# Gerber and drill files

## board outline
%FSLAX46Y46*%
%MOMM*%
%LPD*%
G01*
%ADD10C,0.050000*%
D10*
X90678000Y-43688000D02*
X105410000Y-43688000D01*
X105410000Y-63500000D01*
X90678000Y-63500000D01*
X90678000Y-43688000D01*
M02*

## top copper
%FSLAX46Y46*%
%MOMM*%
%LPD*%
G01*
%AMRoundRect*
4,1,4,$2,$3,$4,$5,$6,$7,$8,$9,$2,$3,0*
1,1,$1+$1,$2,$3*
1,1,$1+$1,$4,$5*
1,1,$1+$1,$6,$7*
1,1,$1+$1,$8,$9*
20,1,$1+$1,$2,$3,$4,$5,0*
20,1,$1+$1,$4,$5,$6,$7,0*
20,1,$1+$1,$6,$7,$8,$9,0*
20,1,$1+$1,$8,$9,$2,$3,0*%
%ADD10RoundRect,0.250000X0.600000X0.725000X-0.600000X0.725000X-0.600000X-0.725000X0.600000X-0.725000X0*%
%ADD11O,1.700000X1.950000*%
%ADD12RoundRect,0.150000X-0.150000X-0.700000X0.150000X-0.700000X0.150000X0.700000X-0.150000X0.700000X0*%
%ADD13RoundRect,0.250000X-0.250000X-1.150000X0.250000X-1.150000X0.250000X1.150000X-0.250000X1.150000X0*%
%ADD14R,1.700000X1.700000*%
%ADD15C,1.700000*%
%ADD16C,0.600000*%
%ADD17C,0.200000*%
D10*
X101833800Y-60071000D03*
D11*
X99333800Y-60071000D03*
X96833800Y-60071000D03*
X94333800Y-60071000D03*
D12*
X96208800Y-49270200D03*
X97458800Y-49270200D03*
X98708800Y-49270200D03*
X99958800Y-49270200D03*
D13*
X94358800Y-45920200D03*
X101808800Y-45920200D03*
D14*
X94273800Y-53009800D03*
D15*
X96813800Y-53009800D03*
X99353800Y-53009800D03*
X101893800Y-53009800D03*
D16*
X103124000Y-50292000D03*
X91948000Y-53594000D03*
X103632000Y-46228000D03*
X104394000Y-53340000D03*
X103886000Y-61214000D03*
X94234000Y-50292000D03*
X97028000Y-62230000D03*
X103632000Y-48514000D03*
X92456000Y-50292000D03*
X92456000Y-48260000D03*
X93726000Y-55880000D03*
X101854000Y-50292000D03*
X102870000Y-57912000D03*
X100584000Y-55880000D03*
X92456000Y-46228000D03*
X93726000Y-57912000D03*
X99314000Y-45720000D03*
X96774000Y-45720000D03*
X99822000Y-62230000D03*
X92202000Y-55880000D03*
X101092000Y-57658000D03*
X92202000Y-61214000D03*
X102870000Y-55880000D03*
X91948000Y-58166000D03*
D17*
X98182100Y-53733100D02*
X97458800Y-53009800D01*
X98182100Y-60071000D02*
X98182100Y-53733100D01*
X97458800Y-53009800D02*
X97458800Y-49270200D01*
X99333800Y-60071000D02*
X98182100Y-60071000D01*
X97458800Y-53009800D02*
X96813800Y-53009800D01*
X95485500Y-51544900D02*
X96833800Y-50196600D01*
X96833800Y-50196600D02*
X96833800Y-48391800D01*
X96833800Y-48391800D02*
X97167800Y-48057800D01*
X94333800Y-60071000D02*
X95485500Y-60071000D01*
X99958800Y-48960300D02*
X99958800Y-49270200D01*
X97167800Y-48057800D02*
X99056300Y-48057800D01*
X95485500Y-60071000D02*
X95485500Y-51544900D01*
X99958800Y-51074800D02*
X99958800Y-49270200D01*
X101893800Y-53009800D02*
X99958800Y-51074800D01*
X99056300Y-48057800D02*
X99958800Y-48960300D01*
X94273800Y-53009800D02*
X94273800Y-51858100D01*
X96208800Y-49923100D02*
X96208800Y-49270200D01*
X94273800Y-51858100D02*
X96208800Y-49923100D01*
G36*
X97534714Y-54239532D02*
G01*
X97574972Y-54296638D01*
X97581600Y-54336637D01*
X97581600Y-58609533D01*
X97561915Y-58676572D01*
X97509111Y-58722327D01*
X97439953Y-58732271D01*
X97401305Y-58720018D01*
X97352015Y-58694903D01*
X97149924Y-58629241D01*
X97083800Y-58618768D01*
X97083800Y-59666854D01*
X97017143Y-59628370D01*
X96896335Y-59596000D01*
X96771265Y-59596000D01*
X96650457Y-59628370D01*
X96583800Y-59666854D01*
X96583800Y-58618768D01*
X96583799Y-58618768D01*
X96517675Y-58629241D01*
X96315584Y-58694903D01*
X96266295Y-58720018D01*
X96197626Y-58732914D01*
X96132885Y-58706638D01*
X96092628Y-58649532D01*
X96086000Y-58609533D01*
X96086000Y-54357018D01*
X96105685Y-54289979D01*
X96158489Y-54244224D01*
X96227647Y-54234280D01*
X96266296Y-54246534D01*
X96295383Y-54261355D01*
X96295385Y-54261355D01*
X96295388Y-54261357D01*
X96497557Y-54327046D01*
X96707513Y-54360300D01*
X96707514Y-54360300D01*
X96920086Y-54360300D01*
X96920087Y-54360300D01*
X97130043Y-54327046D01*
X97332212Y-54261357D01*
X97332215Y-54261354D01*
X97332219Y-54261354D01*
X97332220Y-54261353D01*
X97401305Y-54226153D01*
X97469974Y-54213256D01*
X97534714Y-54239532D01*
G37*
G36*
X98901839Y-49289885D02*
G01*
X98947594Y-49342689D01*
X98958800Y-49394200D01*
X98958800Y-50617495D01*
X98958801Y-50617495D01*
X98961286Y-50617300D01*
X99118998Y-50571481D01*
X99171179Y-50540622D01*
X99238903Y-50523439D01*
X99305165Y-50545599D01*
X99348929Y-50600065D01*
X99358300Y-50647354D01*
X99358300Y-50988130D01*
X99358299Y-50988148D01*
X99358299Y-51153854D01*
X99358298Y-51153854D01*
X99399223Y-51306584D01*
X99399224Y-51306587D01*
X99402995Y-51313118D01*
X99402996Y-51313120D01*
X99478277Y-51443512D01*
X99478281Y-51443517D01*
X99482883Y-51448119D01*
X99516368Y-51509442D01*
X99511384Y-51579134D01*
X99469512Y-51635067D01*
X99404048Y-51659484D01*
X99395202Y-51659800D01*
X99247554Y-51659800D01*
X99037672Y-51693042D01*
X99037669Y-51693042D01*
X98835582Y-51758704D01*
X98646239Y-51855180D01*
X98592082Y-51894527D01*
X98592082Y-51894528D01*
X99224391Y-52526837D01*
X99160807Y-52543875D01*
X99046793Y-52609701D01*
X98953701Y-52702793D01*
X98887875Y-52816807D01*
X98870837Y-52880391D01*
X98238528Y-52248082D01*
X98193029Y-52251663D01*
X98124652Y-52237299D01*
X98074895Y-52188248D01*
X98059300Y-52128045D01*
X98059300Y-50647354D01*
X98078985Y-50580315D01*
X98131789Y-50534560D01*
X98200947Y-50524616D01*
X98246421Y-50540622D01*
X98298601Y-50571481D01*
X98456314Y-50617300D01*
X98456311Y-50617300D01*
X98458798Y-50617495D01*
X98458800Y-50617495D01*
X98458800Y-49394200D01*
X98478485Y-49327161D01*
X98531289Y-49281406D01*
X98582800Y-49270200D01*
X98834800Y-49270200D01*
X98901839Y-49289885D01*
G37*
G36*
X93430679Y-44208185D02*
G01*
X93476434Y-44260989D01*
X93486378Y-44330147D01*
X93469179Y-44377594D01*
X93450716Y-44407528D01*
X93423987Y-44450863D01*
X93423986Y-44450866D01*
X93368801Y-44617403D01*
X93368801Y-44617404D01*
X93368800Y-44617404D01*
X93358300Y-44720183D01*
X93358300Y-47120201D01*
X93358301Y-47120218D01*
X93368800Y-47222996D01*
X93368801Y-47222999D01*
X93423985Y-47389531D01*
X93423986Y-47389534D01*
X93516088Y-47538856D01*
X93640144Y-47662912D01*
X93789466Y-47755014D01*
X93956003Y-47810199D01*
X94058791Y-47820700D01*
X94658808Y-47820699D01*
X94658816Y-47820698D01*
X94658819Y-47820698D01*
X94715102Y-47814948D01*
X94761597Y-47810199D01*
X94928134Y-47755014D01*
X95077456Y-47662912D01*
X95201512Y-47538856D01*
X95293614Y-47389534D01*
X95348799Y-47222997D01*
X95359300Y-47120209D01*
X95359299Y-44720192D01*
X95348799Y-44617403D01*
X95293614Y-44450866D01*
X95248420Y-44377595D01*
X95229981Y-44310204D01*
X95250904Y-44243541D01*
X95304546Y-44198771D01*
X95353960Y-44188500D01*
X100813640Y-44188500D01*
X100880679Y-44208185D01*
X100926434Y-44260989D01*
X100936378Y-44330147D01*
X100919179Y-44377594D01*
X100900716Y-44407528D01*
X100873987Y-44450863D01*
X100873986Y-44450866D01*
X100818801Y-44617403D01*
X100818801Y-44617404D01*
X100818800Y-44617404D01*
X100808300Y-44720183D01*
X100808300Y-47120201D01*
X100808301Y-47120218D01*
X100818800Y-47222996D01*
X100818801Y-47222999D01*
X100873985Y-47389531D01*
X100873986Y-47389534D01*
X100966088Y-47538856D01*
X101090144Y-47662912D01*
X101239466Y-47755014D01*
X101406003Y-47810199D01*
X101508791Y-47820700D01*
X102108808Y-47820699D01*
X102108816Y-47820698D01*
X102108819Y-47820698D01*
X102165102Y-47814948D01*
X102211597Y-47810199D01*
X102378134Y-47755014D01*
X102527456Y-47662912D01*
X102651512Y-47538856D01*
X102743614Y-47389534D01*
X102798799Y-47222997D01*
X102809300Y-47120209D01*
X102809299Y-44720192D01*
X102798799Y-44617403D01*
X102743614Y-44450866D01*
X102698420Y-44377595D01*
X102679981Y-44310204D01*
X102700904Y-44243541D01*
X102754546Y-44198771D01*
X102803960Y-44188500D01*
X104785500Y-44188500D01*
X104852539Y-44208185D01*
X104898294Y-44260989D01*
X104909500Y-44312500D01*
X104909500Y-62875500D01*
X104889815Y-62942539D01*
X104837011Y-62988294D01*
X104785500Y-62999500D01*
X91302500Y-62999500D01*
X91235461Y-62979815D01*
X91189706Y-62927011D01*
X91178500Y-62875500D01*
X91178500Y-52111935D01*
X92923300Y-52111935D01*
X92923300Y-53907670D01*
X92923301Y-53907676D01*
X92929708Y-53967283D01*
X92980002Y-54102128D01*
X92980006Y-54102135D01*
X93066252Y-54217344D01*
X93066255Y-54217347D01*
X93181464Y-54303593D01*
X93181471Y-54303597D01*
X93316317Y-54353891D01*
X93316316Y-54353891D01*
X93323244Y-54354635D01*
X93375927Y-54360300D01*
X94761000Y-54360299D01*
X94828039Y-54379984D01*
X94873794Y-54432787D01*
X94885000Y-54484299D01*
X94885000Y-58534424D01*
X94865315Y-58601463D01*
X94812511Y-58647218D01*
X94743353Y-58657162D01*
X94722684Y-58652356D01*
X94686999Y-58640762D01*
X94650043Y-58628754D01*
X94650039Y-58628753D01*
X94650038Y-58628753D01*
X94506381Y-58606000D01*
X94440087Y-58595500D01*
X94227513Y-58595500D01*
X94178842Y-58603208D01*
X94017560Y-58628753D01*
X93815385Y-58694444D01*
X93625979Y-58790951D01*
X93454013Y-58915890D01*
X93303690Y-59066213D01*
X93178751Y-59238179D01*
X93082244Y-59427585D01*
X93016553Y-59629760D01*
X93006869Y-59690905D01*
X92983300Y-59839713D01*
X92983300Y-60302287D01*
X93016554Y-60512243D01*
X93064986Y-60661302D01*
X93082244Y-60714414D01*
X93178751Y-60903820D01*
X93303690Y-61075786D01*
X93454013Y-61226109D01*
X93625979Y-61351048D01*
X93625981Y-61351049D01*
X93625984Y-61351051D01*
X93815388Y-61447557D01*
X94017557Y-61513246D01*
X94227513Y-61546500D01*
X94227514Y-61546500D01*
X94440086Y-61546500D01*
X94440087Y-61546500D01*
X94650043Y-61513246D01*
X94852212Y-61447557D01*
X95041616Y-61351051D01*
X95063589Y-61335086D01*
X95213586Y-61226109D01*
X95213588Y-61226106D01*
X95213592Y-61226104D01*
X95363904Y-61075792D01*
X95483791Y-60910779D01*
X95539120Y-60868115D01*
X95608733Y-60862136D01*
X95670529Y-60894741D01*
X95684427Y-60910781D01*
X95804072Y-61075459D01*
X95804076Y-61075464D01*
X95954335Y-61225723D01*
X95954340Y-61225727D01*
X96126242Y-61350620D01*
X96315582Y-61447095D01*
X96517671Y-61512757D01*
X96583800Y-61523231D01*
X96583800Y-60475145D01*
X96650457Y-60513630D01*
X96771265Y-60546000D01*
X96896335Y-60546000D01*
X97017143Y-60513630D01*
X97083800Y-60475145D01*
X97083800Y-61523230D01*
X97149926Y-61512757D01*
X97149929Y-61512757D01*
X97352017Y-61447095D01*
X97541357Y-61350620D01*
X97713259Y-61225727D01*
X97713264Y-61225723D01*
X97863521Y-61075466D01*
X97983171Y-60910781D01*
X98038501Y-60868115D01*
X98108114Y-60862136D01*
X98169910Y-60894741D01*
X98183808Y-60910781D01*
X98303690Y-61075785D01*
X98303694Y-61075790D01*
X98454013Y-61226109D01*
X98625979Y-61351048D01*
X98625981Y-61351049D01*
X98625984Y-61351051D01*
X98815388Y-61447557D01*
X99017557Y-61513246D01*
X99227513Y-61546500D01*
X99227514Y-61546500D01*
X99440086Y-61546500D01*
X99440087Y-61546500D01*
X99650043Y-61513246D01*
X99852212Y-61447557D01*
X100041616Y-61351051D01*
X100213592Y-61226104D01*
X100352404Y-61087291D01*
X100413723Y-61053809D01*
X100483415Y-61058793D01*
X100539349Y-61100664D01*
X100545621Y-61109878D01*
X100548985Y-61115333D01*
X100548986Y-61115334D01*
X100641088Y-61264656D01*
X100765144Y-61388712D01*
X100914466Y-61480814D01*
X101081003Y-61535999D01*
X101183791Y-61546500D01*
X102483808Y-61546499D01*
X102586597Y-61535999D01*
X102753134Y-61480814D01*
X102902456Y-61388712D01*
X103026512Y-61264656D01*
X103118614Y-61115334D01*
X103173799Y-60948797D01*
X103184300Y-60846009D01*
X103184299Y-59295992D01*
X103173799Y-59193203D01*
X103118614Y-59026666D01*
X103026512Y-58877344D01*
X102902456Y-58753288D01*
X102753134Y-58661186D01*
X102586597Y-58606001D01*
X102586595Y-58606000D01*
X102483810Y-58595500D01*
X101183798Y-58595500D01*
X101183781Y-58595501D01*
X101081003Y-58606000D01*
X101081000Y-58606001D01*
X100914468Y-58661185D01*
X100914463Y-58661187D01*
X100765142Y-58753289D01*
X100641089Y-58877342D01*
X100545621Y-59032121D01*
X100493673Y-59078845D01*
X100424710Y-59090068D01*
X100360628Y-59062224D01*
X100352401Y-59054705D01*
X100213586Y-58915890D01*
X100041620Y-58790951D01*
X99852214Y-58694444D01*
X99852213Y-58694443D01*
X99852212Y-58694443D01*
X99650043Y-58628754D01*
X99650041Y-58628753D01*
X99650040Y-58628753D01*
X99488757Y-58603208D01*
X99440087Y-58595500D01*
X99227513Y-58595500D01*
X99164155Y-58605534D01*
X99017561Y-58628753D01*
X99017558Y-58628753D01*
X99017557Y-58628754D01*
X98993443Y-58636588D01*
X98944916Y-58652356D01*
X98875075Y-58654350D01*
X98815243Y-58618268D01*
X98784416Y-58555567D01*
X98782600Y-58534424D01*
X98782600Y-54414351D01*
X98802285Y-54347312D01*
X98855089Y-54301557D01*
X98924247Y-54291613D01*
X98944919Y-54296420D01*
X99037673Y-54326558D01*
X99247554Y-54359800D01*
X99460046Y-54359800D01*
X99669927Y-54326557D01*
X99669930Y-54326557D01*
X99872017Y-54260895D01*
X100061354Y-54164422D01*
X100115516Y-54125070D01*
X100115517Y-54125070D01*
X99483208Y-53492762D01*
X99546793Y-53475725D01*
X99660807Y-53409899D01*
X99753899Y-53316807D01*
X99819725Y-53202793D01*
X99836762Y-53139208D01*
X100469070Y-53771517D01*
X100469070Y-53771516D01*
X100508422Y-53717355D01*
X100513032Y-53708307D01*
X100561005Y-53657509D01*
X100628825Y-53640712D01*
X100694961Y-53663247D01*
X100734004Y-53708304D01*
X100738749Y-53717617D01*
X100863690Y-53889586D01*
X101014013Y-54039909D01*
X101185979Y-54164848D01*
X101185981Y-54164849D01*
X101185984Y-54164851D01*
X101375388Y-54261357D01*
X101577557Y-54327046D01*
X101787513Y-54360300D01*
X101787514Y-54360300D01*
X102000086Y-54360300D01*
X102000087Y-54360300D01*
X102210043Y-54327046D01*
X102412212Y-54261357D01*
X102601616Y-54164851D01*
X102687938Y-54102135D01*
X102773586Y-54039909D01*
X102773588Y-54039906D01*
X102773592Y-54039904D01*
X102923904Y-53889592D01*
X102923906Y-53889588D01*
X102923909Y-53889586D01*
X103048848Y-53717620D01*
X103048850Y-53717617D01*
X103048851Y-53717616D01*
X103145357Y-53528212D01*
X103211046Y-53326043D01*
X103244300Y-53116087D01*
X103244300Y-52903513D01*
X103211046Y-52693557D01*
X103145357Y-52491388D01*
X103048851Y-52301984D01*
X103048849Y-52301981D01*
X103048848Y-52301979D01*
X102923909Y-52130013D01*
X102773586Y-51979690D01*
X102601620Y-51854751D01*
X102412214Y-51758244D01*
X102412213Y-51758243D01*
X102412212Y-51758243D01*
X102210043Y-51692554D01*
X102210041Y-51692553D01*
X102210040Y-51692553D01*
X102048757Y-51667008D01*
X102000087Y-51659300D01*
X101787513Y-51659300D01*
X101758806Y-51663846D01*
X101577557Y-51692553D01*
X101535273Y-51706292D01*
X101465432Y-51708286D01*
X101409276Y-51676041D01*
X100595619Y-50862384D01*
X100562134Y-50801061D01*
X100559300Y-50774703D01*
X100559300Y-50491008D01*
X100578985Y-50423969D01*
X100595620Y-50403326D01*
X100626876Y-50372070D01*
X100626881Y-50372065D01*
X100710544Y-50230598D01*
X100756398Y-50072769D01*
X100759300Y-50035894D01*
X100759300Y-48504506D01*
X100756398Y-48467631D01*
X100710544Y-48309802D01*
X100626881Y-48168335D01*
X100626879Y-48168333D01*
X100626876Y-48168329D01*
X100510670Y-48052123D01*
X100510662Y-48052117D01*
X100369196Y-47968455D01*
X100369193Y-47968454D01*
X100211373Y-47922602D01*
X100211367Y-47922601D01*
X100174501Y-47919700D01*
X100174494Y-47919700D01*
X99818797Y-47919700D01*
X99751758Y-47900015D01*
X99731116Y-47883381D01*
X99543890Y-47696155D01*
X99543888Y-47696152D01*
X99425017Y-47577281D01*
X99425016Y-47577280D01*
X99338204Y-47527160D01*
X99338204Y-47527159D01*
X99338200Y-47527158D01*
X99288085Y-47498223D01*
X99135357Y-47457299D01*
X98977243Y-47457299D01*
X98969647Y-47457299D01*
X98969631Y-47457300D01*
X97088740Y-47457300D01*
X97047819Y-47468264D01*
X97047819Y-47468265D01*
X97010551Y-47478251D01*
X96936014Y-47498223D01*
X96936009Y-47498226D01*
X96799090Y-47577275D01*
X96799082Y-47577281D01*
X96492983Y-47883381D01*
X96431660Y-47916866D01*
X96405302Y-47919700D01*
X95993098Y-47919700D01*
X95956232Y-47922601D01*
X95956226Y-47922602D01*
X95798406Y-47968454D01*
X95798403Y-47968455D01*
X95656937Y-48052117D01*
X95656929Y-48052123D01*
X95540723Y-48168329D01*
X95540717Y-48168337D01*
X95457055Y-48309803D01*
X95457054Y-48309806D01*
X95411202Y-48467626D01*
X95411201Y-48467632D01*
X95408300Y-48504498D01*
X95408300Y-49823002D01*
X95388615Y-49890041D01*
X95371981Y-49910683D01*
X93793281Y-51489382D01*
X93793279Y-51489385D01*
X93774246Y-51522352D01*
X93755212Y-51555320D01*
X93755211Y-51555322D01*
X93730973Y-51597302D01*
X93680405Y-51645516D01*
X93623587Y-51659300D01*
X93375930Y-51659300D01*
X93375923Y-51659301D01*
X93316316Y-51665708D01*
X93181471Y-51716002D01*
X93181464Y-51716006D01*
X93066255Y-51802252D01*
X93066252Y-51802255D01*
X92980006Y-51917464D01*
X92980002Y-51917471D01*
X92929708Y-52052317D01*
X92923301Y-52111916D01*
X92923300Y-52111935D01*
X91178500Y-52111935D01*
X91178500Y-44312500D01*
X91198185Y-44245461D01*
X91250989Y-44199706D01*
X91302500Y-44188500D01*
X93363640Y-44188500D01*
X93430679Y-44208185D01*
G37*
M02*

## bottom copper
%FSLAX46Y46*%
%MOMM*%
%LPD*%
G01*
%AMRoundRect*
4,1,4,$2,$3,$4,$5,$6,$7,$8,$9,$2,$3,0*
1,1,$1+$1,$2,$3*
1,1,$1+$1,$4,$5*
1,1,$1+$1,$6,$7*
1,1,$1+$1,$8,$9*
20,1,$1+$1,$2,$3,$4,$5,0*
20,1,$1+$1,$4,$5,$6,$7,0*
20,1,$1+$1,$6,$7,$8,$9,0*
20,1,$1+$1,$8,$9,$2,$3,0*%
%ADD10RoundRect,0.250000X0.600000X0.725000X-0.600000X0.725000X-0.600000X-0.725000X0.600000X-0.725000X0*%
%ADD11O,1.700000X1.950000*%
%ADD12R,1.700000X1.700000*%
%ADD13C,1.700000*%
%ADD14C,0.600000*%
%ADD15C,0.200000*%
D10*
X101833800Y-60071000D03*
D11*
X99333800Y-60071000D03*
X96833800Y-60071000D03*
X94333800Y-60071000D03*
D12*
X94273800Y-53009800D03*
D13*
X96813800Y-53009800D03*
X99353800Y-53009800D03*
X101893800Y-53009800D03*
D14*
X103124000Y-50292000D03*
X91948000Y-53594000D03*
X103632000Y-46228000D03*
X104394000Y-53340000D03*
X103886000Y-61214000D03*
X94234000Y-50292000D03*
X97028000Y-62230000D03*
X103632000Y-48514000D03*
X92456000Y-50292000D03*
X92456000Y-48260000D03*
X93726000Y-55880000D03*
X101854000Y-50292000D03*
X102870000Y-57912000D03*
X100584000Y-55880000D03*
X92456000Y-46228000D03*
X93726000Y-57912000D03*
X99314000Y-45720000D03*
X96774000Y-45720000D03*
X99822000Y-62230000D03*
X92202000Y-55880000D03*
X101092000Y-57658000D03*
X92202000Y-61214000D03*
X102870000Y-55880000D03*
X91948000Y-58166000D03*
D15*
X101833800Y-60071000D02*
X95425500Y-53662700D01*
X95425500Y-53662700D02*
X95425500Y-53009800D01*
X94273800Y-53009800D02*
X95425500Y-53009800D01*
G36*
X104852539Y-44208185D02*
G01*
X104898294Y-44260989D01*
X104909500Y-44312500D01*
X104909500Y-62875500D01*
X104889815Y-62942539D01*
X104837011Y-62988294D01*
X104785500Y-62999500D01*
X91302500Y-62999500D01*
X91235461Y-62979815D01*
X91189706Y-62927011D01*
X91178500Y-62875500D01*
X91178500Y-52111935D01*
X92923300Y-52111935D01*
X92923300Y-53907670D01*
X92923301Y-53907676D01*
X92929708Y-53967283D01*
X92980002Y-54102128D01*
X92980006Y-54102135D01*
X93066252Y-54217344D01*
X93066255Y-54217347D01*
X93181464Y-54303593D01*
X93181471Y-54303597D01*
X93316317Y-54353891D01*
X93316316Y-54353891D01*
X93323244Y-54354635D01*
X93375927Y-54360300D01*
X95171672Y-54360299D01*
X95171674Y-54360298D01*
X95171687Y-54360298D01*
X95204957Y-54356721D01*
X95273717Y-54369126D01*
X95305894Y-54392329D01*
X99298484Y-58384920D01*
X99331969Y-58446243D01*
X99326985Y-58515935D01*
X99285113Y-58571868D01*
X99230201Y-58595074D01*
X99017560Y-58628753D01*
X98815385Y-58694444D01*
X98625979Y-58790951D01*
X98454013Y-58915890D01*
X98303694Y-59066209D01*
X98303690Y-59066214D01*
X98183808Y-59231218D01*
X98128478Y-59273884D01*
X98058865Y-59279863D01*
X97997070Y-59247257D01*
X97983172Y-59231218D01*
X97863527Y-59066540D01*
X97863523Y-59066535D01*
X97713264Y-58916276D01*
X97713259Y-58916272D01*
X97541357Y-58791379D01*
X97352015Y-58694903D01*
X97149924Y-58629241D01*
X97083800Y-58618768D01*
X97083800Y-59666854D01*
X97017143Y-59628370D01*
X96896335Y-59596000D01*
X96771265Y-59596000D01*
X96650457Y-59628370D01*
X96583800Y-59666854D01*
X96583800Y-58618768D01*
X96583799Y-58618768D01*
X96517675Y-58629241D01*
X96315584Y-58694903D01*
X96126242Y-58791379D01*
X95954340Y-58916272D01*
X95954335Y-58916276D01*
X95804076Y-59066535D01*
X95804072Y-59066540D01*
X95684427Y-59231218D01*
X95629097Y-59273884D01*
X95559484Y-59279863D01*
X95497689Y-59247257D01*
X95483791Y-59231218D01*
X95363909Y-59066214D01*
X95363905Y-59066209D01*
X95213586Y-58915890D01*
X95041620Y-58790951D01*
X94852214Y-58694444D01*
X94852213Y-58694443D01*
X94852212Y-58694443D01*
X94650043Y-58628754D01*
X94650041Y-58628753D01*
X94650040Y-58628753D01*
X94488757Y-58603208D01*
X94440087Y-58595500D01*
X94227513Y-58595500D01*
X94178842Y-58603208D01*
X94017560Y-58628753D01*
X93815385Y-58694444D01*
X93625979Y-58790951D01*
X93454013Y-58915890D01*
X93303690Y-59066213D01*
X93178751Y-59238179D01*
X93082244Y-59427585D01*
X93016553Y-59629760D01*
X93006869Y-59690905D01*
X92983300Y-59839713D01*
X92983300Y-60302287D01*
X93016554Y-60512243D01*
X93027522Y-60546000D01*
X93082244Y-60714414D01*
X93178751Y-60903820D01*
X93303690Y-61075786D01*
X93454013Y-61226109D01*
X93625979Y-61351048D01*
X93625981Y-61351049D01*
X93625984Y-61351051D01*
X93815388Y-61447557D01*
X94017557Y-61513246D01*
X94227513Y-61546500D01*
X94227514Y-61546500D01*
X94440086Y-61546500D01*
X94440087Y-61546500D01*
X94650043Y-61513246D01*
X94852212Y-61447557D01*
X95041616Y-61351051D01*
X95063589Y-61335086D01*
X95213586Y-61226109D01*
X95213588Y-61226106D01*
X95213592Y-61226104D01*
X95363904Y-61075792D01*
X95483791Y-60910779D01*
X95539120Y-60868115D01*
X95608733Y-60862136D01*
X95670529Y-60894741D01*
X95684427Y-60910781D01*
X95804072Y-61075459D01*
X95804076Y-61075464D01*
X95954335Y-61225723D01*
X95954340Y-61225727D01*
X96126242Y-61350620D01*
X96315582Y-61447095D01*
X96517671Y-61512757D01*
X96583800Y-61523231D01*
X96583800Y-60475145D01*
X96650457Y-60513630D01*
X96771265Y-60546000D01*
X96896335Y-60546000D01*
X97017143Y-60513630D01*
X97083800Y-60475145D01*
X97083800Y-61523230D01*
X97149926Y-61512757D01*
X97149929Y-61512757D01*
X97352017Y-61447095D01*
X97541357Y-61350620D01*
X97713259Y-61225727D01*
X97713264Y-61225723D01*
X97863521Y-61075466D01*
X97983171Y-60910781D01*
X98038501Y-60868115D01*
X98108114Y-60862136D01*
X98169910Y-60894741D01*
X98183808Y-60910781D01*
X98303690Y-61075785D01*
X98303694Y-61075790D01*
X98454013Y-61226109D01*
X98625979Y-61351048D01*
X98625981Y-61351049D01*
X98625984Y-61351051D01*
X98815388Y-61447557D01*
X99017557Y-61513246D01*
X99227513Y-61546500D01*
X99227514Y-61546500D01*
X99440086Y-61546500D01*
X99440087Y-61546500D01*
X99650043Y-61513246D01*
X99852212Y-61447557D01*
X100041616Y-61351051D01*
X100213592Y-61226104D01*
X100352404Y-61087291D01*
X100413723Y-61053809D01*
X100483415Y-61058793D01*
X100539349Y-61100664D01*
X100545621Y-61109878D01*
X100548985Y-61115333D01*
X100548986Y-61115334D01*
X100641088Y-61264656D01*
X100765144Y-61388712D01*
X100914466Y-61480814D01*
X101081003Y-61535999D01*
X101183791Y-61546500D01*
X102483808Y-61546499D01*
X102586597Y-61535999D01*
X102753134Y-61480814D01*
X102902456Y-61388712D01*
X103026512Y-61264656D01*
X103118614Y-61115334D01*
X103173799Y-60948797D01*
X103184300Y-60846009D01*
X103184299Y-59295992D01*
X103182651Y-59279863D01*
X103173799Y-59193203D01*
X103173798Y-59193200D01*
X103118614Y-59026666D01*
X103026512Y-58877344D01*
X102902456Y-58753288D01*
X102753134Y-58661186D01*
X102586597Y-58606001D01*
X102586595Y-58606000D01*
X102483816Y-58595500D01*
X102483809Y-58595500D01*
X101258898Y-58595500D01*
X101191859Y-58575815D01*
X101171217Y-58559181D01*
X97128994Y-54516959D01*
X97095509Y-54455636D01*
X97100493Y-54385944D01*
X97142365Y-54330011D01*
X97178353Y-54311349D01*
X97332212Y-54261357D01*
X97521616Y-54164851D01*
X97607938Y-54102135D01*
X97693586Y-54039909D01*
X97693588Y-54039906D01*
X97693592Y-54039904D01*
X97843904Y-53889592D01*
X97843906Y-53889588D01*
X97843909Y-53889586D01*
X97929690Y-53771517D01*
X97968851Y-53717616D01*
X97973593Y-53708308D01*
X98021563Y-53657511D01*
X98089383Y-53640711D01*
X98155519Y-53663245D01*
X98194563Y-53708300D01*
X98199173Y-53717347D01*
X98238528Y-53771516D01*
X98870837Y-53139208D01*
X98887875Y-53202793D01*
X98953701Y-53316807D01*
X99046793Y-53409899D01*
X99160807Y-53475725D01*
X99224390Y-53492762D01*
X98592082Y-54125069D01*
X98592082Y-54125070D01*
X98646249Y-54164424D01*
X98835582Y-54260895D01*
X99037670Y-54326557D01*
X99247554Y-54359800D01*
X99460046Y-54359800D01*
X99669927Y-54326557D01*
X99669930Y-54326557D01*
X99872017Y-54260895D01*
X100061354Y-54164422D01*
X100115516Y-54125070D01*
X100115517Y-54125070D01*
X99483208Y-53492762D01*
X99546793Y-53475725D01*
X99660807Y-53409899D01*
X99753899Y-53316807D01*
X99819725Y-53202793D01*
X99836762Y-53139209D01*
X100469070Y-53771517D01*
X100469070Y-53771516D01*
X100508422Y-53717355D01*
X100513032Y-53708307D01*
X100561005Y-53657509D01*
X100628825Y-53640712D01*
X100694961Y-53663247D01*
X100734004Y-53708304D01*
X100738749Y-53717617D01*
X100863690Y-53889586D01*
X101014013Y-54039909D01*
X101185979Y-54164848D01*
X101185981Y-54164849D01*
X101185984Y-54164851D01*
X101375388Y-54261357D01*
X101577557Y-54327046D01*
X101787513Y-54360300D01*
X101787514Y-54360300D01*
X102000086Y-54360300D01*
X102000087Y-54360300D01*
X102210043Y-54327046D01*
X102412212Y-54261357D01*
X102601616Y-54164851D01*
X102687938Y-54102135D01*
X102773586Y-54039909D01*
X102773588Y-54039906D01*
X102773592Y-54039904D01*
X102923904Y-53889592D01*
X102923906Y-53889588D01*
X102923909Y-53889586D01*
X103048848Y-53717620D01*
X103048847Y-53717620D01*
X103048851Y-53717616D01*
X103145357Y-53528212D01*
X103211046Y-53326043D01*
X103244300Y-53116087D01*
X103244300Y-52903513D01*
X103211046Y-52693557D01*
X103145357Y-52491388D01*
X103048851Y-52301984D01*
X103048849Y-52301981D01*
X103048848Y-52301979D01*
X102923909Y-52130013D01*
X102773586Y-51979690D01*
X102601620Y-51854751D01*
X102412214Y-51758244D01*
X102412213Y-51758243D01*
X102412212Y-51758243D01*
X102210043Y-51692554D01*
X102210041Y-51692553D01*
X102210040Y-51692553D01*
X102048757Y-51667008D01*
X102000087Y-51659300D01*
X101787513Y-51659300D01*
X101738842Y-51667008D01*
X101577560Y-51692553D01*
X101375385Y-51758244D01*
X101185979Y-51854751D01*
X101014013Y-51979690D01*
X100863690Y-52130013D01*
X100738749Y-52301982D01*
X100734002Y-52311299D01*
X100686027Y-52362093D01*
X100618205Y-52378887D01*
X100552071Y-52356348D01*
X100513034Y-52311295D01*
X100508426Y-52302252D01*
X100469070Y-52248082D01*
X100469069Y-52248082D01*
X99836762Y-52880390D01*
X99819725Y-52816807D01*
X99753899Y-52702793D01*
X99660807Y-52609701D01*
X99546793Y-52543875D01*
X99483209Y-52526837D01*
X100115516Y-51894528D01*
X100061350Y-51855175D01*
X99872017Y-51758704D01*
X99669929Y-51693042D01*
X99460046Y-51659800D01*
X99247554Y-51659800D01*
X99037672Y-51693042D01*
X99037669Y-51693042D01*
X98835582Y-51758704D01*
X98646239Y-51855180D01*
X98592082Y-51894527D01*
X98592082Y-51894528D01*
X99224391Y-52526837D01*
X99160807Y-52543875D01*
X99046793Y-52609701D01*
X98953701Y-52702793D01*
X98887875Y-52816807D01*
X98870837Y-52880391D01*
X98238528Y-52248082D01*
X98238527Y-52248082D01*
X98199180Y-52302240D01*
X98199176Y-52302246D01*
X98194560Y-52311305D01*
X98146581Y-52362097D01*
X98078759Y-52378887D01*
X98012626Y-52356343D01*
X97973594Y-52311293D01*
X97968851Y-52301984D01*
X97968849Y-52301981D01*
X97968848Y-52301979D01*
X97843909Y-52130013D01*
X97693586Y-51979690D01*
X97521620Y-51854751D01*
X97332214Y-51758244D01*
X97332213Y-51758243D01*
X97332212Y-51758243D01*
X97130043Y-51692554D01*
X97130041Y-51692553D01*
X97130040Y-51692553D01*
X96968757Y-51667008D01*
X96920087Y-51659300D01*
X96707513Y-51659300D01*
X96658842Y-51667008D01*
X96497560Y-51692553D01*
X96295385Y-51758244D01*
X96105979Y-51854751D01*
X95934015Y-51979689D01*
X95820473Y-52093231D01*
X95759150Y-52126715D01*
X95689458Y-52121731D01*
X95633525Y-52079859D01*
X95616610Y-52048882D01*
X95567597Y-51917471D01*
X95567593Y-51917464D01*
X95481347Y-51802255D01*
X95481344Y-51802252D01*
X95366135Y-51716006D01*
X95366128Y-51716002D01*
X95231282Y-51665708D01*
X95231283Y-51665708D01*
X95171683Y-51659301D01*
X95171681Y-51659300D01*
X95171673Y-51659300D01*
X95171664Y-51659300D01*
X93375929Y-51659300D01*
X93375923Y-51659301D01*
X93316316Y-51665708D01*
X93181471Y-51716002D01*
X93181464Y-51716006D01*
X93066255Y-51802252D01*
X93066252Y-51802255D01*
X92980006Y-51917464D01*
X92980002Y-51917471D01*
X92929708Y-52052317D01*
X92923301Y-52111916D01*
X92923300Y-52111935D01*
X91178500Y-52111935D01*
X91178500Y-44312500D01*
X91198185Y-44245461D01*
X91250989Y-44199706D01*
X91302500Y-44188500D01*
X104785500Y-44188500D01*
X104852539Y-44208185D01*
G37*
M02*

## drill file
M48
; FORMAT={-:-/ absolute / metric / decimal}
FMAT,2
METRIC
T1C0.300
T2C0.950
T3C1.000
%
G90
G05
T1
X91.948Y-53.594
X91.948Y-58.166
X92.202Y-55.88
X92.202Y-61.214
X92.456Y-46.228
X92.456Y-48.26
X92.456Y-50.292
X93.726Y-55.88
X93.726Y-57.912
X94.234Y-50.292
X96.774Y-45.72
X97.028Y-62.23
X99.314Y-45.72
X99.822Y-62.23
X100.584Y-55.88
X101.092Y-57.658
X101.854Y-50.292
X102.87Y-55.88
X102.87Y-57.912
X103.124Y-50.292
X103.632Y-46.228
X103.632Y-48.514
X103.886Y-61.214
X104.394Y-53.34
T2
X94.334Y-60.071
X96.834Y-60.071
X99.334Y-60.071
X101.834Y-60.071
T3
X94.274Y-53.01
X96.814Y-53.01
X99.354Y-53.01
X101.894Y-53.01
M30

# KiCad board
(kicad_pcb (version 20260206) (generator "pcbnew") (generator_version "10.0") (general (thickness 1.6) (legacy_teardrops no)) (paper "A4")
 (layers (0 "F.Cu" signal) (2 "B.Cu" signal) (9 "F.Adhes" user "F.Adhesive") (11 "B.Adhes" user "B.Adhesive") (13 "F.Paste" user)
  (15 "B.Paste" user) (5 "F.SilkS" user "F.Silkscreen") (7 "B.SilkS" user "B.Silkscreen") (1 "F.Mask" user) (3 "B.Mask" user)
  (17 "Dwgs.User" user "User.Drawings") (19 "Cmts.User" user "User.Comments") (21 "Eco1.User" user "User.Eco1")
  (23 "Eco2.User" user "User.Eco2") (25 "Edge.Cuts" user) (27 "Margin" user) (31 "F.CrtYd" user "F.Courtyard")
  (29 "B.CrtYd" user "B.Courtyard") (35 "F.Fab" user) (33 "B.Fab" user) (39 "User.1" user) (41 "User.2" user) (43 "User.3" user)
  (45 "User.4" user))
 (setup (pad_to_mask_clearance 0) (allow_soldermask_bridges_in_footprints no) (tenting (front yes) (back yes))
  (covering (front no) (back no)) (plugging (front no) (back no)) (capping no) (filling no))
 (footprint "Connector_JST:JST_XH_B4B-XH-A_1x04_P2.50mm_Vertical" (layer "F.Cu") (at 101.8338 60.071 180)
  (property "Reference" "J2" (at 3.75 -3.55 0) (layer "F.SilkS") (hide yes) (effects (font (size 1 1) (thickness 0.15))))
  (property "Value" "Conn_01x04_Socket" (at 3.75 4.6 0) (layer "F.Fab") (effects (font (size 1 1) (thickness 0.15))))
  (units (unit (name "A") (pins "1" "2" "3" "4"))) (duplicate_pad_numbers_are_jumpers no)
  (pad "1" thru_hole roundrect (at 0 0 180) (size 1.7 1.95) (drill 0.95) (layers "*.Cu" "*.Mask") (remove_unused_layers no)
   (roundrect_rratio 0.147059) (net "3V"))
  (pad "2" thru_hole oval (at 2.5 0 180) (size 1.7 1.95) (drill 0.95) (layers "*.Cu" "*.Mask") (remove_unused_layers no) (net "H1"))
  (pad "3" thru_hole oval (at 5 0 180) (size 1.7 1.95) (drill 0.95) (layers "*.Cu" "*.Mask") (remove_unused_layers no) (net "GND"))
  (pad "4" thru_hole oval (at 7.5 0 180) (size 1.7 1.95) (drill 0.95) (layers "*.Cu" "*.Mask") (remove_unused_layers no) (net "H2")))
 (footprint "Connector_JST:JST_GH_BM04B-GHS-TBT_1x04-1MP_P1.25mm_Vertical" (layer "F.Cu") (at 98.0838 47.3202)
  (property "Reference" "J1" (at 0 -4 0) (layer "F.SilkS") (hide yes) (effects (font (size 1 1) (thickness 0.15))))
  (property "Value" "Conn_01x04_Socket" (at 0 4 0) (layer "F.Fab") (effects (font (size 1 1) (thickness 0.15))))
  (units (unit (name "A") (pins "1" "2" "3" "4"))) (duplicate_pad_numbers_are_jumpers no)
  (pad "1" smd roundrect (at -1.875 1.95) (size 0.6 1.7) (layers "F.Cu" "F.Mask" "F.Paste") (roundrect_rratio 0.25) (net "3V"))
  (pad "2" smd roundrect (at -0.625 1.95) (size 0.6 1.7) (layers "F.Cu" "F.Mask" "F.Paste") (roundrect_rratio 0.25) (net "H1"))
  (pad "3" smd roundrect (at 0.625 1.95) (size 0.6 1.7) (layers "F.Cu" "F.Mask" "F.Paste") (roundrect_rratio 0.25) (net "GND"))
  (pad "4" smd roundrect (at 1.875 1.95) (size 0.6 1.7) (layers "F.Cu" "F.Mask" "F.Paste") (roundrect_rratio 0.25) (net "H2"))
  (pad "MP" smd roundrect (at -3.725 -1.4) (size 1 2.8) (layers "F.Cu" "F.Mask" "F.Paste") (roundrect_rratio 0.25))
  (pad "MP" smd roundrect (at 3.725 -1.4) (size 1 2.8) (layers "F.Cu" "F.Mask" "F.Paste") (roundrect_rratio 0.25)))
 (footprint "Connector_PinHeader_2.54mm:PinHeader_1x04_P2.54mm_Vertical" (layer "F.Cu") (at 94.2738 53.0098 90)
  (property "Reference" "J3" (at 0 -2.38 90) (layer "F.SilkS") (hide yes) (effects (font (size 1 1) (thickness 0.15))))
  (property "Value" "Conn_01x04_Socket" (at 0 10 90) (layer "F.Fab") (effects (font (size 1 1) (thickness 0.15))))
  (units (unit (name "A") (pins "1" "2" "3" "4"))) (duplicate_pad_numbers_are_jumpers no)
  (pad "1" thru_hole rect (at 0 0 90) (size 1.7 1.7) (drill 1) (layers "*.Cu" "*.Mask") (remove_unused_layers no) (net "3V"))
  (pad "2" thru_hole circle (at 0 2.54 90) (size 1.7 1.7) (drill 1) (layers "*.Cu" "*.Mask") (remove_unused_layers no) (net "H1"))
  (pad "3" thru_hole circle (at 0 5.08 90) (size 1.7 1.7) (drill 1) (layers "*.Cu" "*.Mask") (remove_unused_layers no) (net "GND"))
  (pad "4" thru_hole circle (at 0 7.62 90) (size 1.7 1.7) (drill 1) (layers "*.Cu" "*.Mask") (remove_unused_layers no) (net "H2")))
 (gr_rect (start 90.678 43.688) (end 105.41 63.5) (stroke (width 0.05) (type default)) (fill no) (layer "Edge.Cuts"))
 (segment (start 98.1821 53.7331) (end 97.4588 53.0098) (width 0.2) (layer "F.Cu") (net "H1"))
 (segment (start 98.1821 60.071) (end 98.1821 53.7331) (width 0.2) (layer "F.Cu") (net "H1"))
 (segment (start 97.4588 53.0098) (end 97.4588 49.2702) (width 0.2) (layer "F.Cu") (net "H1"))
 (segment (start 99.3338 60.071) (end 98.1821 60.071) (width 0.2) (layer "F.Cu") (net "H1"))
 (segment (start 97.4588 53.0098) (end 96.8138 53.0098) (width 0.2) (layer "F.Cu") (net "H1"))
 (via (at 103.124 50.292) (size 0.6) (drill 0.3) (layers "F.Cu" "B.Cu") (free yes) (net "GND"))
 (via (at 91.948 53.594) (size 0.6) (drill 0.3) (layers "F.Cu" "B.Cu") (free yes) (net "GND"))
 (via (at 103.632 46.228) (size 0.6) (drill 0.3) (layers "F.Cu" "B.Cu") (free yes) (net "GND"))
 (via (at 104.394 53.34) (size 0.6) (drill 0.3) (layers "F.Cu" "B.Cu") (free yes) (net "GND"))
 (via (at 103.886 61.214) (size 0.6) (drill 0.3) (layers "F.Cu" "B.Cu") (free yes) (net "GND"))
 (via (at 94.234 50.292) (size 0.6) (drill 0.3) (layers "F.Cu" "B.Cu") (free yes) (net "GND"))
 (via (at 97.028 62.23) (size 0.6) (drill 0.3) (layers "F.Cu" "B.Cu") (free yes) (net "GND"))
 (via (at 103.632 48.514) (size 0.6) (drill 0.3) (layers "F.Cu" "B.Cu") (free yes) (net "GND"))
 (via (at 92.456 50.292) (size 0.6) (drill 0.3) (layers "F.Cu" "B.Cu") (free yes) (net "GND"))
 (via (at 92.456 48.26) (size 0.6) (drill 0.3) (layers "F.Cu" "B.Cu") (free yes) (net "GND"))
 (via (at 93.726 55.88) (size 0.6) (drill 0.3) (layers "F.Cu" "B.Cu") (free yes) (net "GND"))
 (via (at 101.854 50.292) (size 0.6) (drill 0.3) (layers "F.Cu" "B.Cu") (free yes) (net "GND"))
 (via (at 102.87 57.912) (size 0.6) (drill 0.3) (layers "F.Cu" "B.Cu") (free yes) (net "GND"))
 (via (at 100.584 55.88) (size 0.6) (drill 0.3) (layers "F.Cu" "B.Cu") (free yes) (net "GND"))
 (via (at 92.456 46.228) (size 0.6) (drill 0.3) (layers "F.Cu" "B.Cu") (free yes) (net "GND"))
 (via (at 93.726 57.912) (size 0.6) (drill 0.3) (layers "F.Cu" "B.Cu") (free yes) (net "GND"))
 (via (at 99.314 45.72) (size 0.6) (drill 0.3) (layers "F.Cu" "B.Cu") (free yes) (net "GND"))
 (via (at 96.774 45.72) (size 0.6) (drill 0.3) (layers "F.Cu" "B.Cu") (free yes) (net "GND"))
 (via (at 99.822 62.23) (size 0.6) (drill 0.3) (layers "F.Cu" "B.Cu") (free yes) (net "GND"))
 (via (at 92.202 55.88) (size 0.6) (drill 0.3) (layers "F.Cu" "B.Cu") (free yes) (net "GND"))
 (via (at 101.092 57.658) (size 0.6) (drill 0.3) (layers "F.Cu" "B.Cu") (free yes) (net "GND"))
 (via (at 92.202 61.214) (size 0.6) (drill 0.3) (layers "F.Cu" "B.Cu") (free yes) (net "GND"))
 (via (at 102.87 55.88) (size 0.6) (drill 0.3) (layers "F.Cu" "B.Cu") (free yes) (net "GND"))
 (via (at 91.948 58.166) (size 0.6) (drill 0.3) (layers "F.Cu" "B.Cu") (free yes) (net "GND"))
 (segment (start 95.4855 51.5449) (end 96.8338 50.1966) (width 0.2) (layer "F.Cu") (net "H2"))
 (segment (start 96.8338 50.1966) (end 96.8338 48.3918) (width 0.2) (layer "F.Cu") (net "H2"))
 (segment (start 96.8338 48.3918) (end 97.1678 48.0578) (width 0.2) (layer "F.Cu") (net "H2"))
 (segment (start 94.3338 60.071) (end 95.4855 60.071) (width 0.2) (layer "F.Cu") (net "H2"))
 (segment (start 99.9588 48.9603) (end 99.9588 49.2702) (width 0.2) (layer "F.Cu") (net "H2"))
 (segment (start 97.1678 48.0578) (end 99.0563 48.0578) (width 0.2) (layer "F.Cu") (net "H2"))
 (segment (start 95.4855 60.071) (end 95.4855 51.5449) (width 0.2) (layer "F.Cu") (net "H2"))
 (segment (start 99.9588 51.0748) (end 99.9588 49.2702) (width 0.2) (layer "F.Cu") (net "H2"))
 (segment (start 101.8938 53.0098) (end 99.9588 51.0748) (width 0.2) (layer "F.Cu") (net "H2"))
 (segment (start 99.0563 48.0578) (end 99.9588 48.9603) (width 0.2) (layer "F.Cu") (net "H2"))
 (segment (start 94.2738 53.0098) (end 94.2738 51.8581) (width 0.2) (layer "F.Cu") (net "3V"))
 (segment (start 96.2088 49.9231) (end 96.2088 49.2702) (width 0.2) (layer "F.Cu") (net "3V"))
 (segment (start 94.2738 51.8581) (end 96.2088 49.9231) (width 0.2) (layer "F.Cu") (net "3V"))
 (segment (start 101.8338 60.071) (end 95.4255 53.6627) (width 0.2) (layer "B.Cu") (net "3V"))
 (segment (start 95.4255 53.6627) (end 95.4255 53.0098) (width 0.2) (layer "B.Cu") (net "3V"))
 (segment (start 94.2738 53.0098) (end 95.4255 53.0098) (width 0.2) (layer "B.Cu") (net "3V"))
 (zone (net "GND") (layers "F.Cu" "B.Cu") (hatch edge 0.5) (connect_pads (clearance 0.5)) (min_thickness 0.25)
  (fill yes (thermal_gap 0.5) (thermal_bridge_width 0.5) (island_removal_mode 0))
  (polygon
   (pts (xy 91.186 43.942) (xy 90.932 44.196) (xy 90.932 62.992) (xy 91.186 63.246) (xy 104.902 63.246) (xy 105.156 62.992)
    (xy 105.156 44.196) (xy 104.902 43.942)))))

